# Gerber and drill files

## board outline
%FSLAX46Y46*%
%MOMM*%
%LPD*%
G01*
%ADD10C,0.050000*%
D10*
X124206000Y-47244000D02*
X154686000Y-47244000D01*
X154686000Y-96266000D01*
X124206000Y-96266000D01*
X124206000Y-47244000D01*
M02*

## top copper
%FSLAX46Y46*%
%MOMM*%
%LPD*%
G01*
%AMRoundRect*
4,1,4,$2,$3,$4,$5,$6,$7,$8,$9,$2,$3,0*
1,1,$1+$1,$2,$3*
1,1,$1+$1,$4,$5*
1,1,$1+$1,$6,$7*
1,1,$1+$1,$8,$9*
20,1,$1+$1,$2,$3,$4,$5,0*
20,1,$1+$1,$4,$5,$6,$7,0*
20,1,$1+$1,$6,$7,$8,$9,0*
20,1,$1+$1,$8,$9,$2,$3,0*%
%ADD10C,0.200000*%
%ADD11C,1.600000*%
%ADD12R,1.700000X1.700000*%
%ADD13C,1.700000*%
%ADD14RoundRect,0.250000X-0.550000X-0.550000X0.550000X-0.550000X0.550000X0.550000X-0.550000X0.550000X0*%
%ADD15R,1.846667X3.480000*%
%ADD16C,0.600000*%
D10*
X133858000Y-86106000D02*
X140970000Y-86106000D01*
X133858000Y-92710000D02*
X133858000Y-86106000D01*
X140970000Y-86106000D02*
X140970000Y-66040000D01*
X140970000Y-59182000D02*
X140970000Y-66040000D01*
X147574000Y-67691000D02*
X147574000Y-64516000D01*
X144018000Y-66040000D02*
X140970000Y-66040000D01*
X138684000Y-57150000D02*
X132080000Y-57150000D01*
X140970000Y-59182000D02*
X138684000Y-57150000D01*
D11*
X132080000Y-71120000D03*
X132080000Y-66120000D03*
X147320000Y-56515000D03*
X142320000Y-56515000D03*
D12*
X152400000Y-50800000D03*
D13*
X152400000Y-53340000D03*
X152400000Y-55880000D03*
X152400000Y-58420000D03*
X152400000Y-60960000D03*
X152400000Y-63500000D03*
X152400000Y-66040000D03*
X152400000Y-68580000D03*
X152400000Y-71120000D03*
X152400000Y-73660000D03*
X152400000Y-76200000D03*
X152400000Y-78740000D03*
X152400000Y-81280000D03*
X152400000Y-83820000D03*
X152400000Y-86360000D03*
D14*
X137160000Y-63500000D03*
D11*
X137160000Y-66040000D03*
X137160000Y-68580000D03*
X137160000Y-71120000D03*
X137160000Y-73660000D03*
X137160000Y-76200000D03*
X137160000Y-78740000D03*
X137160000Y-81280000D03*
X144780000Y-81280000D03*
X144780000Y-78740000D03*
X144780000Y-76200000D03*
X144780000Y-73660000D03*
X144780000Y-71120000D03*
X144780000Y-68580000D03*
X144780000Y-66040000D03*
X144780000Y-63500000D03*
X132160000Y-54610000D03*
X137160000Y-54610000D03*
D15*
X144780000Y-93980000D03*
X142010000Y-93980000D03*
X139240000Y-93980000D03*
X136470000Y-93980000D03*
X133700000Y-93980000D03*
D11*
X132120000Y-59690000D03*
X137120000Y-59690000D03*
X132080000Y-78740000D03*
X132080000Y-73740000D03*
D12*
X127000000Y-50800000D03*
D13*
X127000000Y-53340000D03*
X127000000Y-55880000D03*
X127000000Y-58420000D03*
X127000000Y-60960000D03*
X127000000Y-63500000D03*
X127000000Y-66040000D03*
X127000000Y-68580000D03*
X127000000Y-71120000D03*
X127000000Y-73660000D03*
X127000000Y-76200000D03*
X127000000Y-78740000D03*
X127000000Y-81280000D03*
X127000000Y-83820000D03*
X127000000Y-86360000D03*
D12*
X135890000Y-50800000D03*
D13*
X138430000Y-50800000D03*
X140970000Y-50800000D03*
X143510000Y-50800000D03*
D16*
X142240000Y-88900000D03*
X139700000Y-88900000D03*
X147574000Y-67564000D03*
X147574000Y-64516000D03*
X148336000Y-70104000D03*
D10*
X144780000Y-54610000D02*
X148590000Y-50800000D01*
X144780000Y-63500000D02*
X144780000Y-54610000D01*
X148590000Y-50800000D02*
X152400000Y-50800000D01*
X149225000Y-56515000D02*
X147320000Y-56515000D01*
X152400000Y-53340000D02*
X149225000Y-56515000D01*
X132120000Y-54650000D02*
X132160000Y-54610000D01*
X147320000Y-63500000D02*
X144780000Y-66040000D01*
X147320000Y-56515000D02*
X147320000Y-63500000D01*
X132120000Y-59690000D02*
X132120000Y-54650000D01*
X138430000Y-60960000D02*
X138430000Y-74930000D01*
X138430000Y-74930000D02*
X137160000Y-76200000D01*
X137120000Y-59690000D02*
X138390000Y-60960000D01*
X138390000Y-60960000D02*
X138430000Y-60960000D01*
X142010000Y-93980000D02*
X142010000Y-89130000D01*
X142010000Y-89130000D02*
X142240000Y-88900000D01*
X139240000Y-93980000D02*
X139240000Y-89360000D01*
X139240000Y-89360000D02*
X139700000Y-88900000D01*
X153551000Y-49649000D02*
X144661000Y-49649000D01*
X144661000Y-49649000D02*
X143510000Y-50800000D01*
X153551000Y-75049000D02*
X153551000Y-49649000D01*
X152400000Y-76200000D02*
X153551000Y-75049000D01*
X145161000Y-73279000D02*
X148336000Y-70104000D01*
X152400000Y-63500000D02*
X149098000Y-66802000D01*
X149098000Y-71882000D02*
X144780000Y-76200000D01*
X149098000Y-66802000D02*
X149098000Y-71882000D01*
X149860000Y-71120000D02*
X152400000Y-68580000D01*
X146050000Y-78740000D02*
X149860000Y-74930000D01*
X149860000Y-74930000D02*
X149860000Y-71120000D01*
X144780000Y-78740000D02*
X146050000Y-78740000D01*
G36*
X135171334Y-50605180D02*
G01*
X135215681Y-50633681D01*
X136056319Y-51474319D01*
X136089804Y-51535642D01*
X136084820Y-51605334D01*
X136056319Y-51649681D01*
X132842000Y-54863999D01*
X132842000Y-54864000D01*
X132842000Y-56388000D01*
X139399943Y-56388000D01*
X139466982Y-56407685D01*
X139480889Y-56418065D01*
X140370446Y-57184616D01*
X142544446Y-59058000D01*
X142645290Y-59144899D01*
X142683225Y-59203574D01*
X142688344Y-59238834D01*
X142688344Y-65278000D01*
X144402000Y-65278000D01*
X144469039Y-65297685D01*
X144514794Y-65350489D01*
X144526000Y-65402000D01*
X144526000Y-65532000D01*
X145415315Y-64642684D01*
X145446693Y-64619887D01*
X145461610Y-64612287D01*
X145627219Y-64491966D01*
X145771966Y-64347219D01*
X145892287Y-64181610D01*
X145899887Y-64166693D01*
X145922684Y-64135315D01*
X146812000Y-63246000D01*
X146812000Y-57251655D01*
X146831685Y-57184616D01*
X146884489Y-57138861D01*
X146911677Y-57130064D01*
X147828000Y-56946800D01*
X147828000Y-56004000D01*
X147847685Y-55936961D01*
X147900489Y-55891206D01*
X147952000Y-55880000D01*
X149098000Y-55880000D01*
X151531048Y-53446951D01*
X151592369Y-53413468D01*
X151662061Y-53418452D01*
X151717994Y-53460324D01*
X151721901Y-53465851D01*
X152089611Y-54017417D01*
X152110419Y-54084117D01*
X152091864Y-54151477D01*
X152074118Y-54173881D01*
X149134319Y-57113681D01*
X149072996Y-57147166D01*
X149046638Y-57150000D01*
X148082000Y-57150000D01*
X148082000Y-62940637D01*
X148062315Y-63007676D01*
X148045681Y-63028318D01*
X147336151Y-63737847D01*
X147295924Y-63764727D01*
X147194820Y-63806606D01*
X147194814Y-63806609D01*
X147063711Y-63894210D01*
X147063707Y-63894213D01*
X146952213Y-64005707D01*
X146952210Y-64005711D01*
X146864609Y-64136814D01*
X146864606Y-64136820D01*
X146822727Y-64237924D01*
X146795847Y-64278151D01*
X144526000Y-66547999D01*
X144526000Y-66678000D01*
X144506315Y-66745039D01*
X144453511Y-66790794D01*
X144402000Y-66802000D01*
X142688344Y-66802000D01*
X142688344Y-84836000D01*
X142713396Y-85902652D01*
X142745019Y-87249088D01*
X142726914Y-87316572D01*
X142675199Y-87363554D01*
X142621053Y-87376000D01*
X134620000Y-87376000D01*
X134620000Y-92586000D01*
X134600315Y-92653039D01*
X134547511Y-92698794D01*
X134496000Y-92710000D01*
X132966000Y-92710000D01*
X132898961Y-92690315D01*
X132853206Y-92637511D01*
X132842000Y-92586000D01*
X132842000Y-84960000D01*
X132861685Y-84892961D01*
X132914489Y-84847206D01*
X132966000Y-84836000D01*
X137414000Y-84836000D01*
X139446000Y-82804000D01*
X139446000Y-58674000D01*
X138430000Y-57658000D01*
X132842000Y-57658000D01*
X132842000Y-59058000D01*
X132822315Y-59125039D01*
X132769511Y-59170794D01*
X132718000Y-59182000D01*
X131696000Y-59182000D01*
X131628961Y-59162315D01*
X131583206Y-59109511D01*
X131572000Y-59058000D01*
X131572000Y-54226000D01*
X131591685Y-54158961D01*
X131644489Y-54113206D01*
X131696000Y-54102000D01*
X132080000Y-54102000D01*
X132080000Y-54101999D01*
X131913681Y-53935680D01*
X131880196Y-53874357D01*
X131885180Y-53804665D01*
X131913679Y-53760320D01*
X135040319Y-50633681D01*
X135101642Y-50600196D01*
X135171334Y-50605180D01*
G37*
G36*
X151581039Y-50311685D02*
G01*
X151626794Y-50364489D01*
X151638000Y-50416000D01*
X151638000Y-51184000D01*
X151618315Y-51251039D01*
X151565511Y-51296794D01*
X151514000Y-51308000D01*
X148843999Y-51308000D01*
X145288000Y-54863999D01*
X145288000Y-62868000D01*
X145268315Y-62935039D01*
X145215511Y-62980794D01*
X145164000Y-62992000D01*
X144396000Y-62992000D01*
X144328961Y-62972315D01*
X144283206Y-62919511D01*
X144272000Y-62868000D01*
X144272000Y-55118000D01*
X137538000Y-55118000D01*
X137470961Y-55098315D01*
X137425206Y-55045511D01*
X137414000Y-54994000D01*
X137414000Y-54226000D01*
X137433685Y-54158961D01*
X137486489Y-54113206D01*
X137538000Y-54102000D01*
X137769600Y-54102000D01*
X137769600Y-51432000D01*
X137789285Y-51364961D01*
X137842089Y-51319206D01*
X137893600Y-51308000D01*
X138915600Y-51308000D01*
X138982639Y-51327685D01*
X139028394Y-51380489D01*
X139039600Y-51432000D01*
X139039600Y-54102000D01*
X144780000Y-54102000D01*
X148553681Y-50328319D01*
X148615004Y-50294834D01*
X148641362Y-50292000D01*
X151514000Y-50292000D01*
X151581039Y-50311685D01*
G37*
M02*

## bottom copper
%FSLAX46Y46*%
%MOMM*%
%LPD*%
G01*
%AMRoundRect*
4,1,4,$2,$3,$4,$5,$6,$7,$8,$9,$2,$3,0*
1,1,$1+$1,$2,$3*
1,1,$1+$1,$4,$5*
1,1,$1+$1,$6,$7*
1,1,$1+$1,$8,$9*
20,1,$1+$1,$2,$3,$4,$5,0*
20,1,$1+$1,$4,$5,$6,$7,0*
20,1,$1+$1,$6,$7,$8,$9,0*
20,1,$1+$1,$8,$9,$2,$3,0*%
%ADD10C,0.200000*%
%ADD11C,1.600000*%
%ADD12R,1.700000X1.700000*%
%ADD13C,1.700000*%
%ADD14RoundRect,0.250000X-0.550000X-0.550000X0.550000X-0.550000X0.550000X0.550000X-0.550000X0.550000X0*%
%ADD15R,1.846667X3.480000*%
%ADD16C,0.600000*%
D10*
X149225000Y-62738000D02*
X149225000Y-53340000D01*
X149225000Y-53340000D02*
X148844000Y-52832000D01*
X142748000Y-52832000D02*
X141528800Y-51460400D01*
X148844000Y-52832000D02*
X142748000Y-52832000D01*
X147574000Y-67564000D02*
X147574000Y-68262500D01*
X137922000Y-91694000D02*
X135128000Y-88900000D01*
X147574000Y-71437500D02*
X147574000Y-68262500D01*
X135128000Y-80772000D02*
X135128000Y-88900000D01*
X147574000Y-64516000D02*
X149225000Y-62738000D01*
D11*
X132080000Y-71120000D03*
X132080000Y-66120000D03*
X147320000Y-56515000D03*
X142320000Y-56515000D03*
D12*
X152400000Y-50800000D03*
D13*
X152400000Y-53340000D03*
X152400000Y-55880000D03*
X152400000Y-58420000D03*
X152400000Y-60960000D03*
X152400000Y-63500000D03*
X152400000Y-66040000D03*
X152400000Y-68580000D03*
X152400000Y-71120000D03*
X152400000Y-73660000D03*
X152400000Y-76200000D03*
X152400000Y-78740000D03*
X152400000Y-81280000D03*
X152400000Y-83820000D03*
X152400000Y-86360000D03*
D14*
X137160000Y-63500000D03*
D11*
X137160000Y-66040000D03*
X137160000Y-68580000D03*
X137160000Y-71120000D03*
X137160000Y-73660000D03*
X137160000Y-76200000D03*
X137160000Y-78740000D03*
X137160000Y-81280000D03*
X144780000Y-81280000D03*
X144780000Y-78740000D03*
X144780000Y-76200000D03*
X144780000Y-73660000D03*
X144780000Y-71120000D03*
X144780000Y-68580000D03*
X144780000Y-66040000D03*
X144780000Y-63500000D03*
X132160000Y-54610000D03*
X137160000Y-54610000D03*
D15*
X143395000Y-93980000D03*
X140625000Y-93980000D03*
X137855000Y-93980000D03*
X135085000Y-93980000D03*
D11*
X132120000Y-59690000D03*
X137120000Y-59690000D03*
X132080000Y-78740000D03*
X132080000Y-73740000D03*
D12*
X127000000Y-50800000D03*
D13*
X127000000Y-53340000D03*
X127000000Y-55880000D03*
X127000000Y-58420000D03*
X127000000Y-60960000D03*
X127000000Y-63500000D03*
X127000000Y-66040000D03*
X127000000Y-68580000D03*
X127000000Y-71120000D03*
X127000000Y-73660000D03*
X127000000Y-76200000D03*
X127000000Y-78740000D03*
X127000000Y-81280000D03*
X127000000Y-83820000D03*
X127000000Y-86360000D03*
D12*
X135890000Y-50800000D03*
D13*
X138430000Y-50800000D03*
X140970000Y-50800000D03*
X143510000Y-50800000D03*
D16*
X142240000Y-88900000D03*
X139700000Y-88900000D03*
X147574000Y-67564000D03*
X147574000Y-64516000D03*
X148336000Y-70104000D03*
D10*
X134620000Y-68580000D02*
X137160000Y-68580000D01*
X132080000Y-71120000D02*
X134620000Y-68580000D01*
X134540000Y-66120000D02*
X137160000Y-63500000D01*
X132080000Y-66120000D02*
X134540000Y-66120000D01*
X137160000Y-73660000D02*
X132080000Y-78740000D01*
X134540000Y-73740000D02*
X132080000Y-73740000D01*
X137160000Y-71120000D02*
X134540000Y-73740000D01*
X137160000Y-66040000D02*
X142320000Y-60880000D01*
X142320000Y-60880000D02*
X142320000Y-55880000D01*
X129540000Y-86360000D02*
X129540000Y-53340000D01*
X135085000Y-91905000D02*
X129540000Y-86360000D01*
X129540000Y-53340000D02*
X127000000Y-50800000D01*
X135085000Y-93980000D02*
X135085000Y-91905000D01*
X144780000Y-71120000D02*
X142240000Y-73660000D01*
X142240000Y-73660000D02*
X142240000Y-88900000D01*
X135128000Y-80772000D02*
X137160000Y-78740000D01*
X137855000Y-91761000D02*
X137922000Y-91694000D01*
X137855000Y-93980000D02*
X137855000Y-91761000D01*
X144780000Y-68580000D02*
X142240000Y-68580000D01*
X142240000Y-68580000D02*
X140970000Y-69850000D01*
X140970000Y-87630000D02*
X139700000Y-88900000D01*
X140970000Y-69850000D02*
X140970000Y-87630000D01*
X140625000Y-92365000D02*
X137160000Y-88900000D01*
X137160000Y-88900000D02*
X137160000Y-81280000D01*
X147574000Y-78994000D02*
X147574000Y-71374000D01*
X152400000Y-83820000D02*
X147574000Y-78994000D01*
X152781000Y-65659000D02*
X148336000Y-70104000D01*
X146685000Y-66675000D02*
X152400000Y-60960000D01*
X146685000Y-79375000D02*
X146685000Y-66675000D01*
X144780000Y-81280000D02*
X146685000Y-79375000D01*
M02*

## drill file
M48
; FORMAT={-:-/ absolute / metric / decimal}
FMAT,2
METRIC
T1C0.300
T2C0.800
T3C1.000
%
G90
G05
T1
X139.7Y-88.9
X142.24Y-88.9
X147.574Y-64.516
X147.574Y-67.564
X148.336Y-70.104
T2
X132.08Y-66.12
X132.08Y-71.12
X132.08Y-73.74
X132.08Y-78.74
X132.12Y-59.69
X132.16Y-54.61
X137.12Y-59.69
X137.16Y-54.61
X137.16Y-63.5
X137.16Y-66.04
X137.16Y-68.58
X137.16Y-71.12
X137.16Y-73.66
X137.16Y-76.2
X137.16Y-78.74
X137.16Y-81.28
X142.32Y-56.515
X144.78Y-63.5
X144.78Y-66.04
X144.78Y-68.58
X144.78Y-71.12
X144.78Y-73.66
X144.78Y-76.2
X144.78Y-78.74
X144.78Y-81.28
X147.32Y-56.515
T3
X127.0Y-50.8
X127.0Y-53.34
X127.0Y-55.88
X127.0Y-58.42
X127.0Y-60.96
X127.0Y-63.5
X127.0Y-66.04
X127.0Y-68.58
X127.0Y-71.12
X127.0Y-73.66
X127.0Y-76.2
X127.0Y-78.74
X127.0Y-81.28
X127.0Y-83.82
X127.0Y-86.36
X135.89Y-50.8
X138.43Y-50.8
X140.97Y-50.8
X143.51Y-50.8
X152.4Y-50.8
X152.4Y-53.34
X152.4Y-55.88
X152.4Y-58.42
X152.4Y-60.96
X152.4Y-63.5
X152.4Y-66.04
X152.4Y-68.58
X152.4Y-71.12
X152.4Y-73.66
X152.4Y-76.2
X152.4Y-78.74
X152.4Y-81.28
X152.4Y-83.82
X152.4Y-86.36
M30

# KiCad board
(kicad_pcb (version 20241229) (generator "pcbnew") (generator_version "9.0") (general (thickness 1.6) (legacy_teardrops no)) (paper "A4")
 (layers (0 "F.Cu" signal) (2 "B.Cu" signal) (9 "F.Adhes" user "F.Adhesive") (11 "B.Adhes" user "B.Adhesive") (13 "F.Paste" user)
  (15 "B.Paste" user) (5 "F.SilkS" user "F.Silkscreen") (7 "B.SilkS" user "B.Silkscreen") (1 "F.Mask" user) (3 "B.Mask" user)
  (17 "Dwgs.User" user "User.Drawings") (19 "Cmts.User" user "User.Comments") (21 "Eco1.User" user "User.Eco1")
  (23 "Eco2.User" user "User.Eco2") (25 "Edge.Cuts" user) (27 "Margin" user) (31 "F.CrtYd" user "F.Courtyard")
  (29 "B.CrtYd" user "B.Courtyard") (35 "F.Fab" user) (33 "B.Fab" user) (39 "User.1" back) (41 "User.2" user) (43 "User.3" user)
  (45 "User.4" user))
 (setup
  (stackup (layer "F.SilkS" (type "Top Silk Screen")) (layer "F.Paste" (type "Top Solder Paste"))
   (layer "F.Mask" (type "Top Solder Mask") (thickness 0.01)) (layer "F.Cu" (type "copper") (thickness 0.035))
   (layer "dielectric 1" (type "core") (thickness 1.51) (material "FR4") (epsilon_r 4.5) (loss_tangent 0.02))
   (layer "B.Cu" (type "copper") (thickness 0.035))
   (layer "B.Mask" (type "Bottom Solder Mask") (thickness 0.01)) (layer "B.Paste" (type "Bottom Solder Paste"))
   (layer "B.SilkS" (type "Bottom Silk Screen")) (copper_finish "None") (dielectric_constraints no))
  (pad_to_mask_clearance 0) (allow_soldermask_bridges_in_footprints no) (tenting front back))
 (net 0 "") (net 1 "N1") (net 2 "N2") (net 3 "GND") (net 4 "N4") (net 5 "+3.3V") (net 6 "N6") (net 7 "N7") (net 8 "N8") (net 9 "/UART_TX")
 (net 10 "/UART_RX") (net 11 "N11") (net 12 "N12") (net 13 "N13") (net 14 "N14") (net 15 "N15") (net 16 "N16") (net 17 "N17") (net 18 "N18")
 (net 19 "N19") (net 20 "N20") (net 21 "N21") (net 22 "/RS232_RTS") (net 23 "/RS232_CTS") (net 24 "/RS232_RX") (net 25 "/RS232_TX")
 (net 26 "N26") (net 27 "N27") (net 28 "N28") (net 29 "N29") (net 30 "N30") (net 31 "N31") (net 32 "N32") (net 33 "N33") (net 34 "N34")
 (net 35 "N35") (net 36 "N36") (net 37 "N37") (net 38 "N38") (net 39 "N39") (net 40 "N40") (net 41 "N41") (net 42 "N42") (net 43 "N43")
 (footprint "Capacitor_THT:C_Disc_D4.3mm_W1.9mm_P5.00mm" (layer "F.Cu") (at 132.08 71.12 90)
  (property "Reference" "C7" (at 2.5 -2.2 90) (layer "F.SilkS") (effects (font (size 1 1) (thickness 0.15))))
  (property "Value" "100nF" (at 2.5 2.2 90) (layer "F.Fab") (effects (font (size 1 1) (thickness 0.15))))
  (pad "1" thru_hole circle (at 0 0 90) (size 1.6 1.6) (drill 0.8) (layers "*.Cu" "*.Mask") (remove_unused_layers no) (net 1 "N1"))
  (pad "2" thru_hole circle (at 5 0 90) (size 1.6 1.6) (drill 0.8) (layers "*.Cu" "*.Mask") (remove_unused_layers no) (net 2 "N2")))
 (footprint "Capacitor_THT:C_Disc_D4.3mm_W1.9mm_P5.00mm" (layer "F.Cu") (at 147.32 56.515 180)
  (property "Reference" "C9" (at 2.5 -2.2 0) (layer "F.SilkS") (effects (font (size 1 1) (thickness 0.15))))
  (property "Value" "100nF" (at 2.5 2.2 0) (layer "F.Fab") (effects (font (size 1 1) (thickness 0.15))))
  (pad "1" thru_hole circle (at 0 0 180) (size 1.6 1.6) (drill 0.8) (layers "*.Cu" "*.Mask") (remove_unused_layers no) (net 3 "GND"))
  (pad "2" thru_hole circle (at 5 0 180) (size 1.6 1.6) (drill 0.8) (layers "*.Cu" "*.Mask") (remove_unused_layers no) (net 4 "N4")))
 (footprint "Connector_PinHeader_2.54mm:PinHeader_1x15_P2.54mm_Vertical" (layer "F.Cu") (at 152.4 50.8)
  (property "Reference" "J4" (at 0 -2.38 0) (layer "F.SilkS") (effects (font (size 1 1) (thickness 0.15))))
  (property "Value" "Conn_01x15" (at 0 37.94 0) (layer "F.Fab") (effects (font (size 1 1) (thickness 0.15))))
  (pad "1" thru_hole rect (at 0 0) (size 1.7 1.7) (drill 1) (layers "*.Cu" "*.Mask") (remove_unused_layers no) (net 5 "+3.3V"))
  (pad "2" thru_hole circle (at 0 2.54) (size 1.7 1.7) (drill 1) (layers "*.Cu" "*.Mask") (remove_unused_layers no) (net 3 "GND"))
  (pad "3" thru_hole circle (at 0 5.08) (size 1.7 1.7) (drill 1) (layers "*.Cu" "*.Mask") (remove_unused_layers no) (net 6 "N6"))
  (pad "4" thru_hole circle (at 0 7.62) (size 1.7 1.7) (drill 1) (layers "*.Cu" "*.Mask") (remove_unused_layers no) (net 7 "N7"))
  (pad "5" thru_hole circle (at 0 10.16) (size 1.7 1.7) (drill 1) (layers "*.Cu" "*.Mask") (remove_unused_layers no) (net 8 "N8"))
  (pad "6" thru_hole circle (at 0 12.7) (size 1.7 1.7) (drill 1) (layers "*.Cu" "*.Mask") (remove_unused_layers no) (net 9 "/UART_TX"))
  (pad "7" thru_hole circle (at 0 15.24) (size 1.7 1.7) (drill 1) (layers "*.Cu" "*.Mask") (remove_unused_layers no) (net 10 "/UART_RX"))
  (pad "8" thru_hole circle (at 0 17.78) (size 1.7 1.7) (drill 1) (layers "*.Cu" "*.Mask") (remove_unused_layers no) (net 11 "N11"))
  (pad "9" thru_hole circle (at 0 20.32) (size 1.7 1.7) (drill 1) (layers "*.Cu" "*.Mask") (remove_unused_layers no) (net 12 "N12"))
  (pad "10" thru_hole circle (at 0 22.86) (size 1.7 1.7) (drill 1) (layers "*.Cu" "*.Mask") (remove_unused_layers no) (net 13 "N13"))
  (pad "11" thru_hole circle (at 0 25.4) (size 1.7 1.7) (drill 1) (layers "*.Cu" "*.Mask") (remove_unused_layers no) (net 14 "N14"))
  (pad "12" thru_hole circle (at 0 27.94) (size 1.7 1.7) (drill 1) (layers "*.Cu" "*.Mask") (remove_unused_layers no) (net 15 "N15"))
  (pad "13" thru_hole circle (at 0 30.48) (size 1.7 1.7) (drill 1) (layers "*.Cu" "*.Mask") (remove_unused_layers no) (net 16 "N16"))
  (pad "14" thru_hole circle (at 0 33.02) (size 1.7 1.7) (drill 1) (layers "*.Cu" "*.Mask") (remove_unused_layers no) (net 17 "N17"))
  (pad "15" thru_hole circle (at 0 35.56) (size 1.7 1.7) (drill 1) (layers "*.Cu" "*.Mask") (remove_unused_layers no) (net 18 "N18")))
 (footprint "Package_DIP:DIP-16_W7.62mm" (layer "F.Cu") (at 137.16 63.5)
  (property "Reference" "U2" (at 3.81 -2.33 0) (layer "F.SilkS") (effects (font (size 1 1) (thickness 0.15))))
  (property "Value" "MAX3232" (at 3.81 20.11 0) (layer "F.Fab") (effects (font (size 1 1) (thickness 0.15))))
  (pad "1" thru_hole roundrect (at 0 0) (size 1.6 1.6) (drill 0.8) (layers "*.Cu" "*.Mask") (remove_unused_layers no)
   (roundrect_rratio 0.15625) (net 2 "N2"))
  (pad "2" thru_hole circle (at 0 2.54) (size 1.6 1.6) (drill 0.8) (layers "*.Cu" "*.Mask") (remove_unused_layers no) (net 4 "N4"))
  (pad "3" thru_hole circle (at 0 5.08) (size 1.6 1.6) (drill 0.8) (layers "*.Cu" "*.Mask") (remove_unused_layers no) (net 1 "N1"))
  (pad "4" thru_hole circle (at 0 7.62) (size 1.6 1.6) (drill 0.8) (layers "*.Cu" "*.Mask") (remove_unused_layers no) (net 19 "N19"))
  (pad "5" thru_hole circle (at 0 10.16) (size 1.6 1.6) (drill 0.8) (layers "*.Cu" "*.Mask") (remove_unused_layers no) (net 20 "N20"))
  (pad "6" thru_hole circle (at 0 12.7) (size 1.6 1.6) (drill 0.8) (layers "*.Cu" "*.Mask") (remove_unused_layers no) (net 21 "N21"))
  (pad "7" thru_hole circle (at 0 15.24) (size 1.6 1.6) (drill 0.8) (layers "*.Cu" "*.Mask") (remove_unused_layers no) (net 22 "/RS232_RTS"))
  (pad "8" thru_hole circle (at 0 17.78) (size 1.6 1.6) (drill 0.8) (layers "*.Cu" "*.Mask") (remove_unused_layers no) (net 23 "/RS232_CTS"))
  (pad "9" thru_hole circle (at 7.62 17.78) (size 1.6 1.6) (drill 0.8) (layers "*.Cu" "*.Mask") (remove_unused_layers no) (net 8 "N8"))
  (pad "10" thru_hole circle (at 7.62 15.24) (size 1.6 1.6) (drill 0.8) (layers "*.Cu" "*.Mask") (remove_unused_layers no) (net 11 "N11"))
  (pad "11" thru_hole circle (at 7.62 12.7) (size 1.6 1.6) (drill 0.8) (layers "*.Cu" "*.Mask") (remove_unused_layers no) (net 9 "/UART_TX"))
  (pad "12" thru_hole circle (at 7.62 10.16) (size 1.6 1.6) (drill 0.8) (layers "*.Cu" "*.Mask") (remove_unused_layers no)
   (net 10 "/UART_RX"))
  (pad "13" thru_hole circle (at 7.62 7.62) (size 1.6 1.6) (drill 0.8) (layers "*.Cu" "*.Mask") (remove_unused_layers no)
   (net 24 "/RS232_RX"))
  (pad "14" thru_hole circle (at 7.62 5.08) (size 1.6 1.6) (drill 0.8) (layers "*.Cu" "*.Mask") (remove_unused_layers no)
   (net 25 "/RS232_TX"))
  (pad "15" thru_hole circle (at 7.62 2.54) (size 1.6 1.6) (drill 0.8) (layers "*.Cu" "*.Mask") (remove_unused_layers no) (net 3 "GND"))
  (pad "16" thru_hole circle (at 7.62 0) (size 1.6 1.6) (drill 0.8) (layers "*.Cu" "*.Mask") (remove_unused_layers no) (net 5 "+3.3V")))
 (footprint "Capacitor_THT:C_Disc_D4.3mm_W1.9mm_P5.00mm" (layer "F.Cu") (at 132.16 54.61)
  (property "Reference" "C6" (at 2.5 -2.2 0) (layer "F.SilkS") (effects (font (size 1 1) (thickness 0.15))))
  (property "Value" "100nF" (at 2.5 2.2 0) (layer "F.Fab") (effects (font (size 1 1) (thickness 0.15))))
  (pad "1" thru_hole circle (at 0 0) (size 1.6 1.6) (drill 0.8) (layers "*.Cu" "*.Mask") (remove_unused_layers no) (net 3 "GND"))
  (pad "2" thru_hole circle (at 5 0) (size 1.6 1.6) (drill 0.8) (layers "*.Cu" "*.Mask") (remove_unused_layers no) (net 5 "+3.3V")))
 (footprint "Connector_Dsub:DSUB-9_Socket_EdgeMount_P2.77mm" (layer "F.Cu") (at 139.24 93.98)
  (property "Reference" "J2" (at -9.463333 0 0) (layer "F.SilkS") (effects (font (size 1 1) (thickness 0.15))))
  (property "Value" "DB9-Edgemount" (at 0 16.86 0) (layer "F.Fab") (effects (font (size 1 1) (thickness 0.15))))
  (pad "1" smd rect (at 5.54 0) (size 1.846667 3.48) (layers "F.Cu" "F.Mask" "F.Paste") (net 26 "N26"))
  (pad "2" smd rect (at 2.77 0) (size 1.846667 3.48) (layers "F.Cu" "F.Mask" "F.Paste") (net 24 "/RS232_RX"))
  (pad "3" smd rect (at 0 0) (size 1.846667 3.48) (layers "F.Cu" "F.Mask" "F.Paste") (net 25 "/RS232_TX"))
  (pad "4" smd rect (at -2.77 0) (size 1.846667 3.48) (layers "F.Cu" "F.Mask" "F.Paste") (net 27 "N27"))
  (pad "5" smd rect (at -5.54 0) (size 1.846667 3.48) (layers "F.Cu" "F.Mask" "F.Paste") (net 3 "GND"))
  (pad "6" smd rect (at 4.155 0) (size 1.846667 3.48) (layers "B.Cu" "B.Mask" "B.Paste") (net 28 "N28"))
  (pad "7" smd rect (at 1.385 0) (size 1.846667 3.48) (layers "B.Cu" "B.Mask" "B.Paste") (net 23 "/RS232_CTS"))
  (pad "8" smd rect (at -1.385 0) (size 1.846667 3.48) (layers "B.Cu" "B.Mask" "B.Paste") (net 22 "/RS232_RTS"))
  (pad "9" smd rect (at -4.155 0) (size 1.846667 3.48) (layers "B.Cu" "B.Mask" "B.Paste") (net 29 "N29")))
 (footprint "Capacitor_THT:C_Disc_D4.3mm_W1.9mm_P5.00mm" (layer "F.Cu") (at 132.12 59.69)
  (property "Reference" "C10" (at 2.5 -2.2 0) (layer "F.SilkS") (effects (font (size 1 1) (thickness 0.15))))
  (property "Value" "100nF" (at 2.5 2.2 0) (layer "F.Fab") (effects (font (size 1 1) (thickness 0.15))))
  (pad "1" thru_hole circle (at 0 0) (size 1.6 1.6) (drill 0.8) (layers "*.Cu" "*.Mask") (remove_unused_layers no) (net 3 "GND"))
  (pad "2" thru_hole circle (at 5 0) (size 1.6 1.6) (drill 0.8) (layers "*.Cu" "*.Mask") (remove_unused_layers no) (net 21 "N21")))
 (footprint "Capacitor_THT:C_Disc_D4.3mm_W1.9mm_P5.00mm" (layer "F.Cu") (at 132.08 78.74 90)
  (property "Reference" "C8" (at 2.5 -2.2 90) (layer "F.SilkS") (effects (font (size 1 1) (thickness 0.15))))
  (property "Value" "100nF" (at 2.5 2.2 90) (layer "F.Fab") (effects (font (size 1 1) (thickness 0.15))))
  (pad "1" thru_hole circle (at 0 0 90) (size 1.6 1.6) (drill 0.8) (layers "*.Cu" "*.Mask") (remove_unused_layers no) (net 20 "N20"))
  (pad "2" thru_hole circle (at 5 0 90) (size 1.6 1.6) (drill 0.8) (layers "*.Cu" "*.Mask") (remove_unused_layers no) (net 19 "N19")))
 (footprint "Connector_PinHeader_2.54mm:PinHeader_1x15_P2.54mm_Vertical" (layer "F.Cu") (at 127 50.8)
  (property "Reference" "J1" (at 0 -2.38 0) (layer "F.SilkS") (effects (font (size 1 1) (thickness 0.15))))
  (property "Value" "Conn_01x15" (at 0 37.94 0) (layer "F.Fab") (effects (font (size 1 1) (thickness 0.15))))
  (pad "1" thru_hole rect (at 0 0) (size 1.7 1.7) (drill 1) (layers "*.Cu" "*.Mask") (remove_unused_layers no) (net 29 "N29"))
  (pad "2" thru_hole circle (at 0 2.54) (size 1.7 1.7) (drill 1) (layers "*.Cu" "*.Mask") (remove_unused_layers no) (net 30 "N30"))
  (pad "3" thru_hole circle (at 0 5.08) (size 1.7 1.7) (drill 1) (layers "*.Cu" "*.Mask") (remove_unused_layers no) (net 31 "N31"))
  (pad "4" thru_hole circle (at 0 7.62) (size 1.7 1.7) (drill 1) (layers "*.Cu" "*.Mask") (remove_unused_layers no) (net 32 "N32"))
  (pad "5" thru_hole circle (at 0 10.16) (size 1.7 1.7) (drill 1) (layers "*.Cu" "*.Mask") (remove_unused_layers no) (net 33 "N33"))
  (pad "6" thru_hole circle (at 0 12.7) (size 1.7 1.7) (drill 1) (layers "*.Cu" "*.Mask") (remove_unused_layers no) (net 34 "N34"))
  (pad "7" thru_hole circle (at 0 15.24) (size 1.7 1.7) (drill 1) (layers "*.Cu" "*.Mask") (remove_unused_layers no) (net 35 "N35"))
  (pad "8" thru_hole circle (at 0 17.78) (size 1.7 1.7) (drill 1) (layers "*.Cu" "*.Mask") (remove_unused_layers no) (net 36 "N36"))
  (pad "9" thru_hole circle (at 0 20.32) (size 1.7 1.7) (drill 1) (layers "*.Cu" "*.Mask") (remove_unused_layers no) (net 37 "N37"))
  (pad "10" thru_hole circle (at 0 22.86) (size 1.7 1.7) (drill 1) (layers "*.Cu" "*.Mask") (remove_unused_layers no) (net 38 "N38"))
  (pad "11" thru_hole circle (at 0 25.4) (size 1.7 1.7) (drill 1) (layers "*.Cu" "*.Mask") (remove_unused_layers no) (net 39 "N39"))
  (pad "12" thru_hole circle (at 0 27.94) (size 1.7 1.7) (drill 1) (layers "*.Cu" "*.Mask") (remove_unused_layers no) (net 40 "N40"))
  (pad "13" thru_hole circle (at 0 30.48) (size 1.7 1.7) (drill 1) (layers "*.Cu" "*.Mask") (remove_unused_layers no) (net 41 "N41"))
  (pad "14" thru_hole circle (at 0 33.02) (size 1.7 1.7) (drill 1) (layers "*.Cu" "*.Mask") (remove_unused_layers no) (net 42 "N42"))
  (pad "15" thru_hole circle (at 0 35.56) (size 1.7 1.7) (drill 1) (layers "*.Cu" "*.Mask") (remove_unused_layers no) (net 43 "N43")))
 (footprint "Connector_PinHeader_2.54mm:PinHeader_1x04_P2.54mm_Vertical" (layer "F.Cu") (at 135.89 50.8 90)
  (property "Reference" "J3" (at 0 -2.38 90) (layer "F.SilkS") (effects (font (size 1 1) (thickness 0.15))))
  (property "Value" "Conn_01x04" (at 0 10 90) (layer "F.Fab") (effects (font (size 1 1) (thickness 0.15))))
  (pad "1" thru_hole rect (at 0 0 90) (size 1.7 1.7) (drill 1) (layers "*.Cu" "*.Mask") (remove_unused_layers no) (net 3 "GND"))
  (pad "2" thru_hole circle (at 0 2.54 90) (size 1.7 1.7) (drill 1) (layers "*.Cu" "*.Mask") (remove_unused_layers no) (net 5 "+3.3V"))
  (pad "3" thru_hole circle (at 0 5.08 90) (size 1.7 1.7) (drill 1) (layers "*.Cu" "*.Mask") (remove_unused_layers no) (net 17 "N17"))
  (pad "4" thru_hole circle (at 0 7.62 90) (size 1.7 1.7) (drill 1) (layers "*.Cu" "*.Mask") (remove_unused_layers no) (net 14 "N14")))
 (gr_line (start 133.858 86.106) (end 140.97 86.106) (stroke (width 0.2) (type default)) (layer "F.Cu") (net 3))
 (gr_line (start 133.858 92.71) (end 133.858 86.106) (stroke (width 0.2) (type default)) (layer "F.Cu") (net 3))
 (gr_line (start 140.97 86.106) (end 140.97 66.04) (stroke (width 0.2) (type default)) (layer "F.Cu") (net 3))
 (gr_line (start 140.97 59.182) (end 140.97 66.04) (stroke (width 0.2) (type default)) (layer "F.Cu") (net 3))
 (gr_line (start 147.574 67.691) (end 147.574 64.516) (stroke (width 0.2) (type default)) (layer "F.Cu") (net 17))
 (gr_line (start 144.018 66.04) (end 140.97 66.04) (stroke (width 0.2) (type default)) (layer "F.Cu") (net 3))
 (gr_line (start 138.684 57.15) (end 132.08 57.15) (stroke (width 0.2) (type default)) (layer "F.Cu") (net 3))
 (gr_line (start 140.97 59.182) (end 138.684 57.15) (stroke (width 0.2) (type default)) (layer "F.Cu") (net 3))
 (gr_line (start 149.225 62.738) (end 149.225 53.34) (stroke (width 0.2) (type default)) (layer "B.Cu") (net 17))
 (gr_line (start 149.225 53.34) (end 148.844 52.832) (stroke (width 0.2) (type default)) (layer "B.Cu") (net 17))
 (gr_line (start 142.748 52.832) (end 141.5288 51.4604) (stroke (width 0.2) (type default)) (layer "B.Cu") (net 17))
 (gr_line (start 148.844 52.832) (end 142.748 52.832) (stroke (width 0.2) (type default)) (layer "B.Cu") (net 17))
 (gr_line (start 147.574 67.564) (end 147.574 68.2625) (stroke (width 0.2) (type default)) (layer "B.Cu") (net 17))
 (gr_line (start 137.922 91.694) (end 135.128 88.9) (stroke (width 0.2) (type default)) (layer "B.Cu") (net 22))
 (gr_line (start 147.574 71.4375) (end 147.574 68.2625) (stroke (width 0.2) (type default)) (layer "B.Cu") (net 17))
 (gr_line (start 135.128 80.772) (end 135.128 88.9) (stroke (width 0.2) (type default)) (layer "B.Cu") (net 22))
 (gr_line (start 147.574 64.516) (end 149.225 62.738) (stroke (width 0.2) (type default)) (layer "B.Cu") (net 17))
 (gr_rect (start 124.206 47.244) (end 154.686 96.266) (stroke (width 0.05) (type default)) (fill no) (layer "Edge.Cuts"))
 (segment (start 144.78 54.61) (end 148.59 50.8) (width 0.2) (layer "F.Cu") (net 5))
 (segment (start 144.78 63.5) (end 144.78 54.61) (width 0.2) (layer "F.Cu") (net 5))
 (segment (start 148.59 50.8) (end 152.4 50.8) (width 0.2) (layer "F.Cu") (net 5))
 (segment (start 149.225 56.515) (end 147.32 56.515) (width 0.2) (layer "F.Cu") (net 3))
 (segment (start 152.4 53.34) (end 149.225 56.515) (width 0.2) (layer "F.Cu") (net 3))
 (segment (start 132.12 54.65) (end 132.16 54.61) (width 0.2) (layer "F.Cu") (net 3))
 (segment (start 147.32 63.5) (end 144.78 66.04) (width 0.2) (layer "F.Cu") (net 3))
 (segment (start 147.32 56.515) (end 147.32 63.5) (width 0.2) (layer "F.Cu") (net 3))
 (segment (start 132.12 59.69) (end 132.12 54.65) (width 0.2) (layer "F.Cu") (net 3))
 (segment (start 134.62 68.58) (end 137.16 68.58) (width 0.2) (layer "B.Cu") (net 1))
 (segment (start 132.08 71.12) (end 134.62 68.58) (width 0.2) (layer "B.Cu") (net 1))
 (segment (start 134.54 66.12) (end 137.16 63.5) (width 0.2) (layer "B.Cu") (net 2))
 (segment (start 132.08 66.12) (end 134.54 66.12) (width 0.2) (layer "B.Cu") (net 2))
 (segment (start 137.16 73.66) (end 132.08 78.74) (width 0.2) (layer "B.Cu") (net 20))
 (segment (start 134.54 73.74) (end 132.08 73.74) (width 0.2) (layer "B.Cu") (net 19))
 (segment (start 137.16 71.12) (end 134.54 73.74) (width 0.2) (layer "B.Cu") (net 19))
 (segment (start 137.16 66.04) (end 142.32 60.88) (width 0.2) (layer "B.Cu") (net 4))
 (segment (start 142.32 60.88) (end 142.32 55.88) (width 0.2) (layer "B.Cu") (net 4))
 (segment (start 138.43 60.96) (end 138.43 74.93) (width 0.2) (layer "F.Cu") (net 21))
 (segment (start 138.43 74.93) (end 137.16 76.2) (width 0.2) (layer "F.Cu") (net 21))
 (segment (start 137.12 59.69) (end 138.39 60.96) (width 0.2) (layer "F.Cu") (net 21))
 (segment (start 138.39 60.96) (end 138.43 60.96) (width 0.2) (layer "F.Cu") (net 21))
 (segment (start 129.54 86.36) (end 129.54 53.34) (width 0.2) (layer "B.Cu") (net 29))
 (segment (start 135.085 91.905) (end 129.54 86.36) (width 0.2) (layer "B.Cu") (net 29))
 (segment (start 129.54 53.34) (end 127 50.8) (width 0.2) (layer "B.Cu") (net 29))
 (segment (start 135.085 93.98) (end 135.085 91.905) (width 0.2) (layer "B.Cu") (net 29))
 (segment (start 142.01 93.98) (end 142.01 89.13) (width 0.2) (layer "F.Cu") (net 24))
 (segment (start 142.01 89.13) (end 142.24 88.9) (width 0.2) (layer "F.Cu") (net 24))
 (via (at 142.24 88.9) (size 0.6) (drill 0.3) (layers "F.Cu" "B.Cu") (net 24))
 (segment (start 144.78 71.12) (end 142.24 73.66) (width 0.2) (layer "B.Cu") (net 24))
 (segment (start 142.24 73.66) (end 142.24 88.9) (width 0.2) (layer "B.Cu") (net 24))
 (segment (start 135.128 80.772) (end 137.16 78.74) (width 0.2) (layer "B.Cu") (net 22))
 (segment (start 137.855 91.761) (end 137.922 91.694) (width 0.2) (layer "B.Cu") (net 22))
 (segment (start 137.855 93.98) (end 137.855 91.761) (width 0.2) (layer "B.Cu") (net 22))
 (segment (start 139.24 93.98) (end 139.24 89.36) (width 0.2) (layer "F.Cu") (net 25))
 (segment (start 139.24 89.36) (end 139.7 88.9) (width 0.2) (layer "F.Cu") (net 25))
 (via (at 139.7 88.9) (size 0.6) (drill 0.3) (layers "F.Cu" "B.Cu") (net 25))
 (segment (start 144.78 68.58) (end 142.24 68.58) (width 0.2) (layer "B.Cu") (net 25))
 (segment (start 142.24 68.58) (end 140.97 69.85) (width 0.2) (layer "B.Cu") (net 25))
 (segment (start 140.97 87.63) (end 139.7 88.9) (width 0.2) (layer "B.Cu") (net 25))
 (segment (start 140.97 69.85) (end 140.97 87.63) (width 0.2) (layer "B.Cu") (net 25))
 (segment (start 140.625 92.365) (end 137.16 88.9) (width 0.2) (layer "B.Cu") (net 23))
 (segment (start 137.16 88.9) (end 137.16 81.28) (width 0.2) (layer "B.Cu") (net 23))
 (segment (start 153.551 49.649) (end 144.661 49.649) (width 0.2) (layer "F.Cu") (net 14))
 (segment (start 144.661 49.649) (end 143.51 50.8) (width 0.2) (layer "F.Cu") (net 14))
 (segment (start 153.551 75.049) (end 153.551 49.649) (width 0.2) (layer "F.Cu") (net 14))
 (segment (start 152.4 76.2) (end 153.551 75.049) (width 0.2) (layer "F.Cu") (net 14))
 (via (at 147.574 67.564) (size 0.6) (drill 0.3) (layers "F.Cu" "B.Cu") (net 17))
 (via (at 147.574 64.516) (size 0.6) (drill 0.3) (layers "F.Cu" "B.Cu") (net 17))
 (segment (start 147.574 78.994) (end 147.574 71.374) (width 0.2) (layer "B.Cu") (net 17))
 (segment (start 152.4 83.82) (end 147.574 78.994) (width 0.2) (layer "B.Cu") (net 17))
 (segment (start 145.161 73.279) (end 148.336 70.104) (width 0.2) (layer "F.Cu") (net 10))
 (via (at 148.336 70.104) (size 0.6) (drill 0.3) (layers "F.Cu" "B.Cu") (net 10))
 (segment (start 152.781 65.659) (end 148.336 70.104) (width 0.2) (layer "B.Cu") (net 10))
 (segment (start 152.4 63.5) (end 149.098 66.802) (width 0.2) (layer "F.Cu") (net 9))
 (segment (start 149.098 71.882) (end 144.78 76.2) (width 0.2) (layer "F.Cu") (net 9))
 (segment (start 149.098 66.802) (end 149.098 71.882) (width 0.2) (layer "F.Cu") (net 9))
 (segment (start 146.685 66.675) (end 152.4 60.96) (width 0.2) (layer "B.Cu") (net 8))
 (segment (start 146.685 79.375) (end 146.685 66.675) (width 0.2) (layer "B.Cu") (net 8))
 (segment (start 144.78 81.28) (end 146.685 79.375) (width 0.2) (layer "B.Cu") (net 8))
 (segment (start 149.86 71.12) (end 152.4 68.58) (width 0.2) (layer "F.Cu") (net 11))
 (segment (start 146.05 78.74) (end 149.86 74.93) (width 0.2) (layer "F.Cu") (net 11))
 (segment (start 149.86 74.93) (end 149.86 71.12) (width 0.2) (layer "F.Cu") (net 11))
 (segment (start 144.78 78.74) (end 146.05 78.74) (width 0.2) (layer "F.Cu") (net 11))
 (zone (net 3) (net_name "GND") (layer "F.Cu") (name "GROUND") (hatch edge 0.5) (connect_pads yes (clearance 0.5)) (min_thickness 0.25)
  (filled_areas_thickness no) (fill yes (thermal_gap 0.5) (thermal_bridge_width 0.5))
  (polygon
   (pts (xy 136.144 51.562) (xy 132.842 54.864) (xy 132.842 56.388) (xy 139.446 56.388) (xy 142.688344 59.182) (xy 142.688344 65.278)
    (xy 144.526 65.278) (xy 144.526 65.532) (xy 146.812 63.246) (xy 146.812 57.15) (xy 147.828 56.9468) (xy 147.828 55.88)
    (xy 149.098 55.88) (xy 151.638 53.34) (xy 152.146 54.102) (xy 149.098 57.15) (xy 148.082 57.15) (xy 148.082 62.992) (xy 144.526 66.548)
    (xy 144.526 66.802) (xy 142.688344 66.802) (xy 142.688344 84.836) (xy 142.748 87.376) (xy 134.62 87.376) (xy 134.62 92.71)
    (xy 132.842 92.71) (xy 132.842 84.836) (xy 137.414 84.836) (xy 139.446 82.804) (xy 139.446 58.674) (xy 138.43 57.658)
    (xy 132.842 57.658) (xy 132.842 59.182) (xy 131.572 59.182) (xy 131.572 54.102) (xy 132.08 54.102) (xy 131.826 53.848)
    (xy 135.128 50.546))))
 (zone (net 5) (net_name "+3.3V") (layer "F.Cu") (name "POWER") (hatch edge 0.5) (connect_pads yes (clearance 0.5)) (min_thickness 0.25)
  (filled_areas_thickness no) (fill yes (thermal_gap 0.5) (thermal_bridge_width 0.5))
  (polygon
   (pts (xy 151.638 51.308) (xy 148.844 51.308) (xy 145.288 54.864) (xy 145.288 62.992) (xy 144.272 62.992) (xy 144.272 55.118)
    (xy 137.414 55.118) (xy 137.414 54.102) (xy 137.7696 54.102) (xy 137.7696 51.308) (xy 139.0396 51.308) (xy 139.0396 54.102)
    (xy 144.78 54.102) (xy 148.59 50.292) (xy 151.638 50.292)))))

